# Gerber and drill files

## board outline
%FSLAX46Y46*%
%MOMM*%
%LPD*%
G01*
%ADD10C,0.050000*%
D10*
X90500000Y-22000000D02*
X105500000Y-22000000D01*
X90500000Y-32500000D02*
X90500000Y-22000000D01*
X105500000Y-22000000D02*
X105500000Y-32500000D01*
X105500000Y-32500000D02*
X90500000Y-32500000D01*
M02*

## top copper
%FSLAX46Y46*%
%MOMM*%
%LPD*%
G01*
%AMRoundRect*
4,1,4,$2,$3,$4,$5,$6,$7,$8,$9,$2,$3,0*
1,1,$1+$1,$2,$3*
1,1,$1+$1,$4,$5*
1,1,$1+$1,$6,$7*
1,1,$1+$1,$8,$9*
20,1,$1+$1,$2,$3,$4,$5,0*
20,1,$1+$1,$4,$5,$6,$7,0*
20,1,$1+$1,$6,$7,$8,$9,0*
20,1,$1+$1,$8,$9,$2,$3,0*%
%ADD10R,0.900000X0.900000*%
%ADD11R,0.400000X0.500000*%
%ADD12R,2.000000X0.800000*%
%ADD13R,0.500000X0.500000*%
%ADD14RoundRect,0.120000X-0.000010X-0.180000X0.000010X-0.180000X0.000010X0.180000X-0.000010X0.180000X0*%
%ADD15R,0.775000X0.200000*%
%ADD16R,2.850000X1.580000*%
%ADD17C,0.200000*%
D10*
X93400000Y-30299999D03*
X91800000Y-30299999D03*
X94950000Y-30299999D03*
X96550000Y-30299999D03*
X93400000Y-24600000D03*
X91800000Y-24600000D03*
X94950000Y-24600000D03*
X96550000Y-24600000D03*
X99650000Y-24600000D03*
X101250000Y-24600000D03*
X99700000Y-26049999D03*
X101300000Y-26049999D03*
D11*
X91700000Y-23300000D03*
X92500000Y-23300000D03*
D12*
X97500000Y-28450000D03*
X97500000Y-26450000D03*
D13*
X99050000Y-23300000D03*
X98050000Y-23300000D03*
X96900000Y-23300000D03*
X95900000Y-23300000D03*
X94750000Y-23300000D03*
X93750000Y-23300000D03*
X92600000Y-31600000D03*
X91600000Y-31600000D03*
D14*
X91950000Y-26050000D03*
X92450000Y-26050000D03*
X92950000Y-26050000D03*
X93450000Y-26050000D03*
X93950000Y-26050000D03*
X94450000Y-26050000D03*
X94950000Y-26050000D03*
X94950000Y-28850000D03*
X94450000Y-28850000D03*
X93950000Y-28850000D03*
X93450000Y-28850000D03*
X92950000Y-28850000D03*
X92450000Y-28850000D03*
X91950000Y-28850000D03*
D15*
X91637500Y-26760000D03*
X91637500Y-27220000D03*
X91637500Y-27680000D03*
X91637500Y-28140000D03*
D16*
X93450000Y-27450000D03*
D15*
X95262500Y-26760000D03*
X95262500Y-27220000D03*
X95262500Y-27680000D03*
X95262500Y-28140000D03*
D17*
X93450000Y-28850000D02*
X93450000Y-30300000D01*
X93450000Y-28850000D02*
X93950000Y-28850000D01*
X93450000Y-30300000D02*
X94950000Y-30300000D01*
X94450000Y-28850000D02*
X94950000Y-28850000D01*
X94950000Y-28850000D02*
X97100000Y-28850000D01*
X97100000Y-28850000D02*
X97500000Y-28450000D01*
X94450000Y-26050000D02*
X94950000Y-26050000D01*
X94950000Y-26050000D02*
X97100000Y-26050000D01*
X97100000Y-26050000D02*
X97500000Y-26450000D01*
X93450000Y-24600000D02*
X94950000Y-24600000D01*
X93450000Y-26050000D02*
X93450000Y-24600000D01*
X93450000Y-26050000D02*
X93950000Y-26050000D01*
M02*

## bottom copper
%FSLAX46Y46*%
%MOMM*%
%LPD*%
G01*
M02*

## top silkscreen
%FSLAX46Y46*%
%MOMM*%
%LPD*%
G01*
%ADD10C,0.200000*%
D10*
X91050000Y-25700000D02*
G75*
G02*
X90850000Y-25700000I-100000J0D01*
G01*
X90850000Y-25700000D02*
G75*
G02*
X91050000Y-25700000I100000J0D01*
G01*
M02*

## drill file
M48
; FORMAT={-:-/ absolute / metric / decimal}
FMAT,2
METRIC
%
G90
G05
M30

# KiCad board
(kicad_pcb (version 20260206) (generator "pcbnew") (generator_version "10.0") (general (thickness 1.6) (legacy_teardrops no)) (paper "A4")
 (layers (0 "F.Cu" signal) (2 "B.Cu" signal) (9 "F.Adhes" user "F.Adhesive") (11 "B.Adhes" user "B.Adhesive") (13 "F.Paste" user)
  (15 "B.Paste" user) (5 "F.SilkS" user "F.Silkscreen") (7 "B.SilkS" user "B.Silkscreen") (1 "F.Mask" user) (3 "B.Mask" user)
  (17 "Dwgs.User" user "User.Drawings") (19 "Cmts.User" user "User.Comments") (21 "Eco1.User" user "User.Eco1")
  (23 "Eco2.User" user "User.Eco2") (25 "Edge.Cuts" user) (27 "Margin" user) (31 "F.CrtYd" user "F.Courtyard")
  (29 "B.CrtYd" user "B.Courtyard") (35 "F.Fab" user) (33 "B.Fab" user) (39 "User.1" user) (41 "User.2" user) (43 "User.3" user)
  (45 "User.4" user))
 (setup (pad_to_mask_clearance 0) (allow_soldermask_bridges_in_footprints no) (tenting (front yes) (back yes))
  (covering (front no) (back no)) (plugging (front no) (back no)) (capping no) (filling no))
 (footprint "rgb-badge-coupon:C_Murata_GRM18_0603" (layer "F.Cu") (at 92.6 30.299999 180)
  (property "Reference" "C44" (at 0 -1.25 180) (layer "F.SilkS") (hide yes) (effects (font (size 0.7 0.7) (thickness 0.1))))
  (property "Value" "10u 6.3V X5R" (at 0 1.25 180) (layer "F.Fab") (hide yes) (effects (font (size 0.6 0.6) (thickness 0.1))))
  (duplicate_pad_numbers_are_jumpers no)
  (pad "1" smd rect (at -0.8 0 180) (size 0.9 0.9) (layers "F.Cu" "F.Mask" "F.Paste") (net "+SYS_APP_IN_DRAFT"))
  (pad "2" smd rect (at 0.8 0 180) (size 0.9 0.9) (layers "F.Cu" "F.Mask" "F.Paste") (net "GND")))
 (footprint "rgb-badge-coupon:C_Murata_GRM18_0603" (layer "F.Cu") (at 95.75 30.299999)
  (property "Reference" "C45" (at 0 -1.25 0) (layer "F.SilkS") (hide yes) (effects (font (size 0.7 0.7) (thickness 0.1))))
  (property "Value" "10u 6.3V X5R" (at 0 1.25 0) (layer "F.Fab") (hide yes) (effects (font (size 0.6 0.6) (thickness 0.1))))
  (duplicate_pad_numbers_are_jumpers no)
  (pad "1" smd rect (at -0.8 0) (size 0.9 0.9) (layers "F.Cu" "F.Mask" "F.Paste") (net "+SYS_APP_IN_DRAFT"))
  (pad "2" smd rect (at 0.8 0) (size 0.9 0.9) (layers "F.Cu" "F.Mask" "F.Paste") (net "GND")))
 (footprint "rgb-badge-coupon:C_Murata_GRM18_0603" (layer "F.Cu") (at 92.6 24.6 180)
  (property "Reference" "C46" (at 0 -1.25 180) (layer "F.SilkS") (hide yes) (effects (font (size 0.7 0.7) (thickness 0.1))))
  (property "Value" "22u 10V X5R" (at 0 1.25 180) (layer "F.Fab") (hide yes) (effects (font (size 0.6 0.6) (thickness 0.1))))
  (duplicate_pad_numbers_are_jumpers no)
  (pad "1" smd rect (at -0.8 0 180) (size 0.9 0.9) (layers "F.Cu" "F.Mask" "F.Paste") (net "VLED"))
  (pad "2" smd rect (at 0.8 0 180) (size 0.9 0.9) (layers "F.Cu" "F.Mask" "F.Paste") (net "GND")))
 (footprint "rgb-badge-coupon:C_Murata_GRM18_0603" (layer "F.Cu") (at 95.75 24.6)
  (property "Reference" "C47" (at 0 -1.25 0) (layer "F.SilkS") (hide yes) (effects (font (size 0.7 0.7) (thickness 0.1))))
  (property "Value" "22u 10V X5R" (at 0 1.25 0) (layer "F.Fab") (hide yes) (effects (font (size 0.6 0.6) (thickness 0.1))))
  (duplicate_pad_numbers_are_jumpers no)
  (pad "1" smd rect (at -0.8 0) (size 0.9 0.9) (layers "F.Cu" "F.Mask" "F.Paste") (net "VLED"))
  (pad "2" smd rect (at 0.8 0) (size 0.9 0.9) (layers "F.Cu" "F.Mask" "F.Paste") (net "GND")))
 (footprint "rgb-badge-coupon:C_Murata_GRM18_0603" (layer "F.Cu") (at 100.45 24.6)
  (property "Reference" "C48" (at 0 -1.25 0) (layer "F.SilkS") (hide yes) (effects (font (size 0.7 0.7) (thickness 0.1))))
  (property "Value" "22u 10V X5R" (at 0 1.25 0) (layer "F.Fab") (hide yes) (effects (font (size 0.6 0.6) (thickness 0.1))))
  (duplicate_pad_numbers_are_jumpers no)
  (pad "1" smd rect (at -0.8 0) (size 0.9 0.9) (layers "F.Cu" "F.Mask" "F.Paste") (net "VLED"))
  (pad "2" smd rect (at 0.8 0) (size 0.9 0.9) (layers "F.Cu" "F.Mask" "F.Paste") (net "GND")))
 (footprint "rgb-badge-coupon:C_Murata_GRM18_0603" (layer "F.Cu") (at 100.5 26.049999)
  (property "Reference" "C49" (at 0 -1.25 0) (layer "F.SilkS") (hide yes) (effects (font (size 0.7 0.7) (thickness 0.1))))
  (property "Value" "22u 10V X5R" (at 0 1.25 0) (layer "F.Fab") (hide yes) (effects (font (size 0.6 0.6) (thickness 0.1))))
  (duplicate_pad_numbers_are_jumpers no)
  (pad "1" smd rect (at -0.8 0) (size 0.9 0.9) (layers "F.Cu" "F.Mask" "F.Paste") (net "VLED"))
  (pad "2" smd rect (at 0.8 0) (size 0.9 0.9) (layers "F.Cu" "F.Mask" "F.Paste") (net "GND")))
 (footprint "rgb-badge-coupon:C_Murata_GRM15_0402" (layer "F.Cu") (at 92.1 23.3)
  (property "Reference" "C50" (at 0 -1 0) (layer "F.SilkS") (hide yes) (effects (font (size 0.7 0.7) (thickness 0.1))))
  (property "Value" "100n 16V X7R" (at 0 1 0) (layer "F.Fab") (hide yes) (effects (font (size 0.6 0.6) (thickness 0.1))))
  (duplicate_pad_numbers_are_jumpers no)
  (pad "1" smd rect (at -0.4 0) (size 0.4 0.5) (layers "F.Cu" "F.Mask" "F.Paste") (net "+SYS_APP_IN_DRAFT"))
  (pad "2" smd rect (at 0.4 0) (size 0.4 0.5) (layers "F.Cu" "F.Mask" "F.Paste") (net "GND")))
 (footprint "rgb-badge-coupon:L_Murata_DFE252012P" (layer "F.Cu") (at 97.5 27.45 90)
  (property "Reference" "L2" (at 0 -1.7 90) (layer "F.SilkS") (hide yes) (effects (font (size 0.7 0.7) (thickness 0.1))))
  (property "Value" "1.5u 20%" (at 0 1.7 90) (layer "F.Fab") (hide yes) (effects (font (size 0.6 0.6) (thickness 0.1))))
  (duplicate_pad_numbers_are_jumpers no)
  (pad "1" smd rect (at -1 0 90) (size 0.8 2) (layers "F.Cu" "F.Mask" "F.Paste") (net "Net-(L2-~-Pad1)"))
  (pad "2" smd rect (at 1 0 90) (size 0.8 2) (layers "F.Cu" "F.Mask" "F.Paste") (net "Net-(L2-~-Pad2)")))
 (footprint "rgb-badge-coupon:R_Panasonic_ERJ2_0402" (layer "F.Cu") (at 98.55 23.3 180)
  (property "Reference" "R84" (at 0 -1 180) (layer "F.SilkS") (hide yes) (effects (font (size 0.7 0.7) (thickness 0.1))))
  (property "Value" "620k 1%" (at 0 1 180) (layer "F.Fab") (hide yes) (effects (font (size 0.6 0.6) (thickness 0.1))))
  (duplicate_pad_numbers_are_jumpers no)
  (pad "1" smd rect (at -0.5 0 180) (size 0.5 0.5) (layers "F.Cu" "F.Mask" "F.Paste") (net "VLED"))
  (pad "2" smd rect (at 0.5 0 180) (size 0.5 0.5) (layers "F.Cu" "F.Mask" "F.Paste") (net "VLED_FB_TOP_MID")))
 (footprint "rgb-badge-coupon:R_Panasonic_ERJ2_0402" (layer "F.Cu") (at 96.4 23.3 180)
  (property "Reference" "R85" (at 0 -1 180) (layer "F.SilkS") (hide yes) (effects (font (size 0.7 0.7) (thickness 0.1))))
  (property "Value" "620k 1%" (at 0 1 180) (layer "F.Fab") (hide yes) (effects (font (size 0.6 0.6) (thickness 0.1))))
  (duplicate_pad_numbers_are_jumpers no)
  (pad "1" smd rect (at -0.5 0 180) (size 0.5 0.5) (layers "F.Cu" "F.Mask" "F.Paste") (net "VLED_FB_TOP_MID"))
  (pad "2" smd rect (at 0.5 0 180) (size 0.5 0.5) (layers "F.Cu" "F.Mask" "F.Paste") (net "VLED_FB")))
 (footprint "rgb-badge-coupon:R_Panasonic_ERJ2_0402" (layer "F.Cu") (at 94.25 23.3 180)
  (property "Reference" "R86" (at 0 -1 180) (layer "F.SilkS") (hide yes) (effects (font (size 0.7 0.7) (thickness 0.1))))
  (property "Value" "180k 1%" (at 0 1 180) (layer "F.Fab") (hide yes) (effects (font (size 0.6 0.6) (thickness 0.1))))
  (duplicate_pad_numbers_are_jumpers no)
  (pad "1" smd rect (at -0.5 0 180) (size 0.5 0.5) (layers "F.Cu" "F.Mask" "F.Paste") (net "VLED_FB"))
  (pad "2" smd rect (at 0.5 0 180) (size 0.5 0.5) (layers "F.Cu" "F.Mask" "F.Paste") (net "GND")))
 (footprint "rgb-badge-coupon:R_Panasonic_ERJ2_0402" (layer "F.Cu") (at 92.1 31.6 180)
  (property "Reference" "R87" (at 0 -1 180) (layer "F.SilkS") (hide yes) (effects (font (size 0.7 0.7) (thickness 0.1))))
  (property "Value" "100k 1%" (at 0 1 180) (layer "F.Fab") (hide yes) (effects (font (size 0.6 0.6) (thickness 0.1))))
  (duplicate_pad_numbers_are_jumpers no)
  (pad "1" smd rect (at -0.5 0 180) (size 0.5 0.5) (layers "F.Cu" "F.Mask" "F.Paste") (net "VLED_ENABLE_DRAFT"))
  (pad "2" smd rect (at 0.5 0 180) (size 0.5 0.5) (layers "F.Cu" "F.Mask" "F.Paste") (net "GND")))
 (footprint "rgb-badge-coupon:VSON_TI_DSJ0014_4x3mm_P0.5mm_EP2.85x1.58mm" (layer "F.Cu") (at 93.45 27.45)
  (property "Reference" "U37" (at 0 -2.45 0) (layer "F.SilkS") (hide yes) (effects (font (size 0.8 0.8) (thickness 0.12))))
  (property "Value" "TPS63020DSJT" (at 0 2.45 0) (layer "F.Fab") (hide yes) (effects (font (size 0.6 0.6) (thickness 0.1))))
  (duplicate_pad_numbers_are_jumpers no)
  (fp_circle (center -2.5 -1.75) (end -2.35 -1.75) (stroke (width 0.1) (type default)) (fill yes) (layer "F.SilkS"))
  (pad "" smd rect (at -1.775 -0.69) (size 0.85 0.2) (layers "F.Paste"))
  (pad "" smd rect (at -1.775 -0.23) (size 0.85 0.2) (layers "F.Paste"))
  (pad "" smd rect (at -1.775 0.23) (size 0.85 0.2) (layers "F.Paste"))
  (pad "" smd rect (at -1.775 0.69) (size 0.85 0.2) (layers "F.Paste"))
  (pad "" smd rect (at -0.725 -0.46) (size 1.25 0.66) (layers "F.Paste"))
  (pad "" smd rect (at -0.725 0.46) (size 1.25 0.66) (layers "F.Paste"))
  (pad "" smd rect (at 0.725 -0.46) (size 1.25 0.66) (layers "F.Paste"))
  (pad "" smd rect (at 0.725 0.46) (size 1.25 0.66) (layers "F.Paste"))
  (pad "" smd rect (at 1.775 -0.69) (size 0.85 0.2) (layers "F.Paste"))
  (pad "" smd rect (at 1.775 -0.23) (size 0.85 0.2) (layers "F.Paste"))
  (pad "" smd rect (at 1.775 0.23) (size 0.85 0.2) (layers "F.Paste"))
  (pad "" smd rect (at 1.775 0.69) (size 0.85 0.2) (layers "F.Paste"))
  (pad "1" smd roundrect (at -1.5 -1.4) (size 0.24 0.6) (layers "F.Cu" "F.Mask" "F.Paste") (roundrect_rratio 0.5) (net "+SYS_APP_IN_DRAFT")
   (solder_mask_margin 0.07))
  (pad "2" smd roundrect (at -1 -1.4) (size 0.24 0.6) (layers "F.Cu" "F.Mask" "F.Paste") (roundrect_rratio 0.5) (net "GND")
   (solder_mask_margin 0.07))
  (pad "3" smd roundrect (at -0.5 -1.4) (size 0.24 0.6) (layers "F.Cu" "F.Mask" "F.Paste") (roundrect_rratio 0.5) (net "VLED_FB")
   (solder_mask_margin 0.07))
  (pad "4" smd roundrect (at 0 -1.4) (size 0.24 0.6) (layers "F.Cu" "F.Mask" "F.Paste") (roundrect_rratio 0.5) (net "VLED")
   (solder_mask_margin 0.07))
  (pad "5" smd roundrect (at 0.5 -1.4) (size 0.24 0.6) (layers "F.Cu" "F.Mask" "F.Paste") (roundrect_rratio 0.5) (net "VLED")
   (solder_mask_margin 0.07))
  (pad "6" smd roundrect (at 1 -1.4) (size 0.24 0.6) (layers "F.Cu" "F.Mask" "F.Paste") (roundrect_rratio 0.5) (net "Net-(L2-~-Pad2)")
   (solder_mask_margin 0.07))
  (pad "7" smd roundrect (at 1.5 -1.4) (size 0.24 0.6) (layers "F.Cu" "F.Mask" "F.Paste") (roundrect_rratio 0.5) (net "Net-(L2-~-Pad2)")
   (solder_mask_margin 0.07))
  (pad "8" smd roundrect (at 1.5 1.4) (size 0.24 0.6) (layers "F.Cu" "F.Mask" "F.Paste") (roundrect_rratio 0.5) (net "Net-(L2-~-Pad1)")
   (solder_mask_margin 0.07))
  (pad "9" smd roundrect (at 1 1.4) (size 0.24 0.6) (layers "F.Cu" "F.Mask" "F.Paste") (roundrect_rratio 0.5) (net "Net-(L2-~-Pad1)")
   (solder_mask_margin 0.07))
  (pad "10" smd roundrect (at 0.5 1.4) (size 0.24 0.6) (layers "F.Cu" "F.Mask" "F.Paste") (roundrect_rratio 0.5) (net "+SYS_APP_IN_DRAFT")
   (solder_mask_margin 0.07))
  (pad "11" smd roundrect (at 0 1.4) (size 0.24 0.6) (layers "F.Cu" "F.Mask" "F.Paste") (roundrect_rratio 0.5) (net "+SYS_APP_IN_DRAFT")
   (solder_mask_margin 0.07))
  (pad "12" smd roundrect (at -0.5 1.4) (size 0.24 0.6) (layers "F.Cu" "F.Mask" "F.Paste") (roundrect_rratio 0.5) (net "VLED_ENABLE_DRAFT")
   (solder_mask_margin 0.07))
  (pad "13" smd roundrect (at -1 1.4) (size 0.24 0.6) (layers "F.Cu" "F.Mask" "F.Paste") (roundrect_rratio 0.5) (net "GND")
   (solder_mask_margin 0.07))
  (pad "14" smd roundrect (at -1.5 1.4) (size 0.24 0.6) (layers "F.Cu" "F.Mask" "F.Paste") (roundrect_rratio 0.5) (solder_mask_margin 0.07))
  (pad "15" smd rect (at -1.8125 -0.69) (size 0.775 0.2) (layers "F.Cu" "F.Mask") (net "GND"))
  (pad "15" smd rect (at -1.8125 -0.23) (size 0.775 0.2) (layers "F.Cu" "F.Mask") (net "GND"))
  (pad "15" smd rect (at -1.8125 0.23) (size 0.775 0.2) (layers "F.Cu" "F.Mask") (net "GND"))
  (pad "15" smd rect (at -1.8125 0.69) (size 0.775 0.2) (layers "F.Cu" "F.Mask") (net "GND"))
  (pad "15" smd rect (at 0 0) (size 2.85 1.58) (layers "F.Cu" "F.Mask") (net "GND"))
  (pad "15" smd rect (at 1.8125 -0.69) (size 0.775 0.2) (layers "F.Cu" "F.Mask") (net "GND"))
  (pad "15" smd rect (at 1.8125 -0.23) (size 0.775 0.2) (layers "F.Cu" "F.Mask") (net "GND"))
  (pad "15" smd rect (at 1.8125 0.23) (size 0.775 0.2) (layers "F.Cu" "F.Mask") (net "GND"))
  (pad "15" smd rect (at 1.8125 0.69) (size 0.775 0.2) (layers "F.Cu" "F.Mask") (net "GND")))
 (gr_line (start 90.5 22) (end 105.5 22) (stroke (width 0.05) (type default)) (layer "Edge.Cuts"))
 (gr_line (start 90.5 32.5) (end 90.5 22) (stroke (width 0.05) (type default)) (layer "Edge.Cuts"))
 (gr_line (start 105.5 22) (end 105.5 32.5) (stroke (width 0.05) (type default)) (layer "Edge.Cuts"))
 (gr_line (start 105.5 32.5) (end 90.5 32.5) (stroke (width 0.05) (type default)) (layer "Edge.Cuts"))
 (segment (start 93.45 28.85) (end 93.45 30.3) (width 0.2) (layer "F.Cu") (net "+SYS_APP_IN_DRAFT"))
 (segment (start 93.45 28.85) (end 93.95 28.85) (width 0.2) (layer "F.Cu") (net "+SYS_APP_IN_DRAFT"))
 (segment (start 93.45 30.3) (end 94.95 30.3) (width 0.2) (layer "F.Cu") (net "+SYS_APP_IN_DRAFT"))
 (segment (start 94.45 28.85) (end 94.95 28.85) (width 0.2) (layer "F.Cu") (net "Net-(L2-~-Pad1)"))
 (segment (start 94.95 28.85) (end 97.1 28.85) (width 0.2) (layer "F.Cu") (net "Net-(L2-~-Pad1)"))
 (segment (start 97.1 28.85) (end 97.5 28.45) (width 0.2) (layer "F.Cu") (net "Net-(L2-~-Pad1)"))
 (segment (start 94.45 26.05) (end 94.95 26.05) (width 0.2) (layer "F.Cu") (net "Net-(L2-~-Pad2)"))
 (segment (start 94.95 26.05) (end 97.1 26.05) (width 0.2) (layer "F.Cu") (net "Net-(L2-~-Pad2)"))
 (segment (start 97.1 26.05) (end 97.5 26.45) (width 0.2) (layer "F.Cu") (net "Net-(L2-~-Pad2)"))
 (segment (start 93.45 24.6) (end 94.95 24.6) (width 0.2) (layer "F.Cu") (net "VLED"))
 (segment (start 93.45 26.05) (end 93.45 24.6) (width 0.2) (layer "F.Cu") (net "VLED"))
 (segment (start 93.45 26.05) (end 93.95 26.05) (width 0.2) (layer "F.Cu") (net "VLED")))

